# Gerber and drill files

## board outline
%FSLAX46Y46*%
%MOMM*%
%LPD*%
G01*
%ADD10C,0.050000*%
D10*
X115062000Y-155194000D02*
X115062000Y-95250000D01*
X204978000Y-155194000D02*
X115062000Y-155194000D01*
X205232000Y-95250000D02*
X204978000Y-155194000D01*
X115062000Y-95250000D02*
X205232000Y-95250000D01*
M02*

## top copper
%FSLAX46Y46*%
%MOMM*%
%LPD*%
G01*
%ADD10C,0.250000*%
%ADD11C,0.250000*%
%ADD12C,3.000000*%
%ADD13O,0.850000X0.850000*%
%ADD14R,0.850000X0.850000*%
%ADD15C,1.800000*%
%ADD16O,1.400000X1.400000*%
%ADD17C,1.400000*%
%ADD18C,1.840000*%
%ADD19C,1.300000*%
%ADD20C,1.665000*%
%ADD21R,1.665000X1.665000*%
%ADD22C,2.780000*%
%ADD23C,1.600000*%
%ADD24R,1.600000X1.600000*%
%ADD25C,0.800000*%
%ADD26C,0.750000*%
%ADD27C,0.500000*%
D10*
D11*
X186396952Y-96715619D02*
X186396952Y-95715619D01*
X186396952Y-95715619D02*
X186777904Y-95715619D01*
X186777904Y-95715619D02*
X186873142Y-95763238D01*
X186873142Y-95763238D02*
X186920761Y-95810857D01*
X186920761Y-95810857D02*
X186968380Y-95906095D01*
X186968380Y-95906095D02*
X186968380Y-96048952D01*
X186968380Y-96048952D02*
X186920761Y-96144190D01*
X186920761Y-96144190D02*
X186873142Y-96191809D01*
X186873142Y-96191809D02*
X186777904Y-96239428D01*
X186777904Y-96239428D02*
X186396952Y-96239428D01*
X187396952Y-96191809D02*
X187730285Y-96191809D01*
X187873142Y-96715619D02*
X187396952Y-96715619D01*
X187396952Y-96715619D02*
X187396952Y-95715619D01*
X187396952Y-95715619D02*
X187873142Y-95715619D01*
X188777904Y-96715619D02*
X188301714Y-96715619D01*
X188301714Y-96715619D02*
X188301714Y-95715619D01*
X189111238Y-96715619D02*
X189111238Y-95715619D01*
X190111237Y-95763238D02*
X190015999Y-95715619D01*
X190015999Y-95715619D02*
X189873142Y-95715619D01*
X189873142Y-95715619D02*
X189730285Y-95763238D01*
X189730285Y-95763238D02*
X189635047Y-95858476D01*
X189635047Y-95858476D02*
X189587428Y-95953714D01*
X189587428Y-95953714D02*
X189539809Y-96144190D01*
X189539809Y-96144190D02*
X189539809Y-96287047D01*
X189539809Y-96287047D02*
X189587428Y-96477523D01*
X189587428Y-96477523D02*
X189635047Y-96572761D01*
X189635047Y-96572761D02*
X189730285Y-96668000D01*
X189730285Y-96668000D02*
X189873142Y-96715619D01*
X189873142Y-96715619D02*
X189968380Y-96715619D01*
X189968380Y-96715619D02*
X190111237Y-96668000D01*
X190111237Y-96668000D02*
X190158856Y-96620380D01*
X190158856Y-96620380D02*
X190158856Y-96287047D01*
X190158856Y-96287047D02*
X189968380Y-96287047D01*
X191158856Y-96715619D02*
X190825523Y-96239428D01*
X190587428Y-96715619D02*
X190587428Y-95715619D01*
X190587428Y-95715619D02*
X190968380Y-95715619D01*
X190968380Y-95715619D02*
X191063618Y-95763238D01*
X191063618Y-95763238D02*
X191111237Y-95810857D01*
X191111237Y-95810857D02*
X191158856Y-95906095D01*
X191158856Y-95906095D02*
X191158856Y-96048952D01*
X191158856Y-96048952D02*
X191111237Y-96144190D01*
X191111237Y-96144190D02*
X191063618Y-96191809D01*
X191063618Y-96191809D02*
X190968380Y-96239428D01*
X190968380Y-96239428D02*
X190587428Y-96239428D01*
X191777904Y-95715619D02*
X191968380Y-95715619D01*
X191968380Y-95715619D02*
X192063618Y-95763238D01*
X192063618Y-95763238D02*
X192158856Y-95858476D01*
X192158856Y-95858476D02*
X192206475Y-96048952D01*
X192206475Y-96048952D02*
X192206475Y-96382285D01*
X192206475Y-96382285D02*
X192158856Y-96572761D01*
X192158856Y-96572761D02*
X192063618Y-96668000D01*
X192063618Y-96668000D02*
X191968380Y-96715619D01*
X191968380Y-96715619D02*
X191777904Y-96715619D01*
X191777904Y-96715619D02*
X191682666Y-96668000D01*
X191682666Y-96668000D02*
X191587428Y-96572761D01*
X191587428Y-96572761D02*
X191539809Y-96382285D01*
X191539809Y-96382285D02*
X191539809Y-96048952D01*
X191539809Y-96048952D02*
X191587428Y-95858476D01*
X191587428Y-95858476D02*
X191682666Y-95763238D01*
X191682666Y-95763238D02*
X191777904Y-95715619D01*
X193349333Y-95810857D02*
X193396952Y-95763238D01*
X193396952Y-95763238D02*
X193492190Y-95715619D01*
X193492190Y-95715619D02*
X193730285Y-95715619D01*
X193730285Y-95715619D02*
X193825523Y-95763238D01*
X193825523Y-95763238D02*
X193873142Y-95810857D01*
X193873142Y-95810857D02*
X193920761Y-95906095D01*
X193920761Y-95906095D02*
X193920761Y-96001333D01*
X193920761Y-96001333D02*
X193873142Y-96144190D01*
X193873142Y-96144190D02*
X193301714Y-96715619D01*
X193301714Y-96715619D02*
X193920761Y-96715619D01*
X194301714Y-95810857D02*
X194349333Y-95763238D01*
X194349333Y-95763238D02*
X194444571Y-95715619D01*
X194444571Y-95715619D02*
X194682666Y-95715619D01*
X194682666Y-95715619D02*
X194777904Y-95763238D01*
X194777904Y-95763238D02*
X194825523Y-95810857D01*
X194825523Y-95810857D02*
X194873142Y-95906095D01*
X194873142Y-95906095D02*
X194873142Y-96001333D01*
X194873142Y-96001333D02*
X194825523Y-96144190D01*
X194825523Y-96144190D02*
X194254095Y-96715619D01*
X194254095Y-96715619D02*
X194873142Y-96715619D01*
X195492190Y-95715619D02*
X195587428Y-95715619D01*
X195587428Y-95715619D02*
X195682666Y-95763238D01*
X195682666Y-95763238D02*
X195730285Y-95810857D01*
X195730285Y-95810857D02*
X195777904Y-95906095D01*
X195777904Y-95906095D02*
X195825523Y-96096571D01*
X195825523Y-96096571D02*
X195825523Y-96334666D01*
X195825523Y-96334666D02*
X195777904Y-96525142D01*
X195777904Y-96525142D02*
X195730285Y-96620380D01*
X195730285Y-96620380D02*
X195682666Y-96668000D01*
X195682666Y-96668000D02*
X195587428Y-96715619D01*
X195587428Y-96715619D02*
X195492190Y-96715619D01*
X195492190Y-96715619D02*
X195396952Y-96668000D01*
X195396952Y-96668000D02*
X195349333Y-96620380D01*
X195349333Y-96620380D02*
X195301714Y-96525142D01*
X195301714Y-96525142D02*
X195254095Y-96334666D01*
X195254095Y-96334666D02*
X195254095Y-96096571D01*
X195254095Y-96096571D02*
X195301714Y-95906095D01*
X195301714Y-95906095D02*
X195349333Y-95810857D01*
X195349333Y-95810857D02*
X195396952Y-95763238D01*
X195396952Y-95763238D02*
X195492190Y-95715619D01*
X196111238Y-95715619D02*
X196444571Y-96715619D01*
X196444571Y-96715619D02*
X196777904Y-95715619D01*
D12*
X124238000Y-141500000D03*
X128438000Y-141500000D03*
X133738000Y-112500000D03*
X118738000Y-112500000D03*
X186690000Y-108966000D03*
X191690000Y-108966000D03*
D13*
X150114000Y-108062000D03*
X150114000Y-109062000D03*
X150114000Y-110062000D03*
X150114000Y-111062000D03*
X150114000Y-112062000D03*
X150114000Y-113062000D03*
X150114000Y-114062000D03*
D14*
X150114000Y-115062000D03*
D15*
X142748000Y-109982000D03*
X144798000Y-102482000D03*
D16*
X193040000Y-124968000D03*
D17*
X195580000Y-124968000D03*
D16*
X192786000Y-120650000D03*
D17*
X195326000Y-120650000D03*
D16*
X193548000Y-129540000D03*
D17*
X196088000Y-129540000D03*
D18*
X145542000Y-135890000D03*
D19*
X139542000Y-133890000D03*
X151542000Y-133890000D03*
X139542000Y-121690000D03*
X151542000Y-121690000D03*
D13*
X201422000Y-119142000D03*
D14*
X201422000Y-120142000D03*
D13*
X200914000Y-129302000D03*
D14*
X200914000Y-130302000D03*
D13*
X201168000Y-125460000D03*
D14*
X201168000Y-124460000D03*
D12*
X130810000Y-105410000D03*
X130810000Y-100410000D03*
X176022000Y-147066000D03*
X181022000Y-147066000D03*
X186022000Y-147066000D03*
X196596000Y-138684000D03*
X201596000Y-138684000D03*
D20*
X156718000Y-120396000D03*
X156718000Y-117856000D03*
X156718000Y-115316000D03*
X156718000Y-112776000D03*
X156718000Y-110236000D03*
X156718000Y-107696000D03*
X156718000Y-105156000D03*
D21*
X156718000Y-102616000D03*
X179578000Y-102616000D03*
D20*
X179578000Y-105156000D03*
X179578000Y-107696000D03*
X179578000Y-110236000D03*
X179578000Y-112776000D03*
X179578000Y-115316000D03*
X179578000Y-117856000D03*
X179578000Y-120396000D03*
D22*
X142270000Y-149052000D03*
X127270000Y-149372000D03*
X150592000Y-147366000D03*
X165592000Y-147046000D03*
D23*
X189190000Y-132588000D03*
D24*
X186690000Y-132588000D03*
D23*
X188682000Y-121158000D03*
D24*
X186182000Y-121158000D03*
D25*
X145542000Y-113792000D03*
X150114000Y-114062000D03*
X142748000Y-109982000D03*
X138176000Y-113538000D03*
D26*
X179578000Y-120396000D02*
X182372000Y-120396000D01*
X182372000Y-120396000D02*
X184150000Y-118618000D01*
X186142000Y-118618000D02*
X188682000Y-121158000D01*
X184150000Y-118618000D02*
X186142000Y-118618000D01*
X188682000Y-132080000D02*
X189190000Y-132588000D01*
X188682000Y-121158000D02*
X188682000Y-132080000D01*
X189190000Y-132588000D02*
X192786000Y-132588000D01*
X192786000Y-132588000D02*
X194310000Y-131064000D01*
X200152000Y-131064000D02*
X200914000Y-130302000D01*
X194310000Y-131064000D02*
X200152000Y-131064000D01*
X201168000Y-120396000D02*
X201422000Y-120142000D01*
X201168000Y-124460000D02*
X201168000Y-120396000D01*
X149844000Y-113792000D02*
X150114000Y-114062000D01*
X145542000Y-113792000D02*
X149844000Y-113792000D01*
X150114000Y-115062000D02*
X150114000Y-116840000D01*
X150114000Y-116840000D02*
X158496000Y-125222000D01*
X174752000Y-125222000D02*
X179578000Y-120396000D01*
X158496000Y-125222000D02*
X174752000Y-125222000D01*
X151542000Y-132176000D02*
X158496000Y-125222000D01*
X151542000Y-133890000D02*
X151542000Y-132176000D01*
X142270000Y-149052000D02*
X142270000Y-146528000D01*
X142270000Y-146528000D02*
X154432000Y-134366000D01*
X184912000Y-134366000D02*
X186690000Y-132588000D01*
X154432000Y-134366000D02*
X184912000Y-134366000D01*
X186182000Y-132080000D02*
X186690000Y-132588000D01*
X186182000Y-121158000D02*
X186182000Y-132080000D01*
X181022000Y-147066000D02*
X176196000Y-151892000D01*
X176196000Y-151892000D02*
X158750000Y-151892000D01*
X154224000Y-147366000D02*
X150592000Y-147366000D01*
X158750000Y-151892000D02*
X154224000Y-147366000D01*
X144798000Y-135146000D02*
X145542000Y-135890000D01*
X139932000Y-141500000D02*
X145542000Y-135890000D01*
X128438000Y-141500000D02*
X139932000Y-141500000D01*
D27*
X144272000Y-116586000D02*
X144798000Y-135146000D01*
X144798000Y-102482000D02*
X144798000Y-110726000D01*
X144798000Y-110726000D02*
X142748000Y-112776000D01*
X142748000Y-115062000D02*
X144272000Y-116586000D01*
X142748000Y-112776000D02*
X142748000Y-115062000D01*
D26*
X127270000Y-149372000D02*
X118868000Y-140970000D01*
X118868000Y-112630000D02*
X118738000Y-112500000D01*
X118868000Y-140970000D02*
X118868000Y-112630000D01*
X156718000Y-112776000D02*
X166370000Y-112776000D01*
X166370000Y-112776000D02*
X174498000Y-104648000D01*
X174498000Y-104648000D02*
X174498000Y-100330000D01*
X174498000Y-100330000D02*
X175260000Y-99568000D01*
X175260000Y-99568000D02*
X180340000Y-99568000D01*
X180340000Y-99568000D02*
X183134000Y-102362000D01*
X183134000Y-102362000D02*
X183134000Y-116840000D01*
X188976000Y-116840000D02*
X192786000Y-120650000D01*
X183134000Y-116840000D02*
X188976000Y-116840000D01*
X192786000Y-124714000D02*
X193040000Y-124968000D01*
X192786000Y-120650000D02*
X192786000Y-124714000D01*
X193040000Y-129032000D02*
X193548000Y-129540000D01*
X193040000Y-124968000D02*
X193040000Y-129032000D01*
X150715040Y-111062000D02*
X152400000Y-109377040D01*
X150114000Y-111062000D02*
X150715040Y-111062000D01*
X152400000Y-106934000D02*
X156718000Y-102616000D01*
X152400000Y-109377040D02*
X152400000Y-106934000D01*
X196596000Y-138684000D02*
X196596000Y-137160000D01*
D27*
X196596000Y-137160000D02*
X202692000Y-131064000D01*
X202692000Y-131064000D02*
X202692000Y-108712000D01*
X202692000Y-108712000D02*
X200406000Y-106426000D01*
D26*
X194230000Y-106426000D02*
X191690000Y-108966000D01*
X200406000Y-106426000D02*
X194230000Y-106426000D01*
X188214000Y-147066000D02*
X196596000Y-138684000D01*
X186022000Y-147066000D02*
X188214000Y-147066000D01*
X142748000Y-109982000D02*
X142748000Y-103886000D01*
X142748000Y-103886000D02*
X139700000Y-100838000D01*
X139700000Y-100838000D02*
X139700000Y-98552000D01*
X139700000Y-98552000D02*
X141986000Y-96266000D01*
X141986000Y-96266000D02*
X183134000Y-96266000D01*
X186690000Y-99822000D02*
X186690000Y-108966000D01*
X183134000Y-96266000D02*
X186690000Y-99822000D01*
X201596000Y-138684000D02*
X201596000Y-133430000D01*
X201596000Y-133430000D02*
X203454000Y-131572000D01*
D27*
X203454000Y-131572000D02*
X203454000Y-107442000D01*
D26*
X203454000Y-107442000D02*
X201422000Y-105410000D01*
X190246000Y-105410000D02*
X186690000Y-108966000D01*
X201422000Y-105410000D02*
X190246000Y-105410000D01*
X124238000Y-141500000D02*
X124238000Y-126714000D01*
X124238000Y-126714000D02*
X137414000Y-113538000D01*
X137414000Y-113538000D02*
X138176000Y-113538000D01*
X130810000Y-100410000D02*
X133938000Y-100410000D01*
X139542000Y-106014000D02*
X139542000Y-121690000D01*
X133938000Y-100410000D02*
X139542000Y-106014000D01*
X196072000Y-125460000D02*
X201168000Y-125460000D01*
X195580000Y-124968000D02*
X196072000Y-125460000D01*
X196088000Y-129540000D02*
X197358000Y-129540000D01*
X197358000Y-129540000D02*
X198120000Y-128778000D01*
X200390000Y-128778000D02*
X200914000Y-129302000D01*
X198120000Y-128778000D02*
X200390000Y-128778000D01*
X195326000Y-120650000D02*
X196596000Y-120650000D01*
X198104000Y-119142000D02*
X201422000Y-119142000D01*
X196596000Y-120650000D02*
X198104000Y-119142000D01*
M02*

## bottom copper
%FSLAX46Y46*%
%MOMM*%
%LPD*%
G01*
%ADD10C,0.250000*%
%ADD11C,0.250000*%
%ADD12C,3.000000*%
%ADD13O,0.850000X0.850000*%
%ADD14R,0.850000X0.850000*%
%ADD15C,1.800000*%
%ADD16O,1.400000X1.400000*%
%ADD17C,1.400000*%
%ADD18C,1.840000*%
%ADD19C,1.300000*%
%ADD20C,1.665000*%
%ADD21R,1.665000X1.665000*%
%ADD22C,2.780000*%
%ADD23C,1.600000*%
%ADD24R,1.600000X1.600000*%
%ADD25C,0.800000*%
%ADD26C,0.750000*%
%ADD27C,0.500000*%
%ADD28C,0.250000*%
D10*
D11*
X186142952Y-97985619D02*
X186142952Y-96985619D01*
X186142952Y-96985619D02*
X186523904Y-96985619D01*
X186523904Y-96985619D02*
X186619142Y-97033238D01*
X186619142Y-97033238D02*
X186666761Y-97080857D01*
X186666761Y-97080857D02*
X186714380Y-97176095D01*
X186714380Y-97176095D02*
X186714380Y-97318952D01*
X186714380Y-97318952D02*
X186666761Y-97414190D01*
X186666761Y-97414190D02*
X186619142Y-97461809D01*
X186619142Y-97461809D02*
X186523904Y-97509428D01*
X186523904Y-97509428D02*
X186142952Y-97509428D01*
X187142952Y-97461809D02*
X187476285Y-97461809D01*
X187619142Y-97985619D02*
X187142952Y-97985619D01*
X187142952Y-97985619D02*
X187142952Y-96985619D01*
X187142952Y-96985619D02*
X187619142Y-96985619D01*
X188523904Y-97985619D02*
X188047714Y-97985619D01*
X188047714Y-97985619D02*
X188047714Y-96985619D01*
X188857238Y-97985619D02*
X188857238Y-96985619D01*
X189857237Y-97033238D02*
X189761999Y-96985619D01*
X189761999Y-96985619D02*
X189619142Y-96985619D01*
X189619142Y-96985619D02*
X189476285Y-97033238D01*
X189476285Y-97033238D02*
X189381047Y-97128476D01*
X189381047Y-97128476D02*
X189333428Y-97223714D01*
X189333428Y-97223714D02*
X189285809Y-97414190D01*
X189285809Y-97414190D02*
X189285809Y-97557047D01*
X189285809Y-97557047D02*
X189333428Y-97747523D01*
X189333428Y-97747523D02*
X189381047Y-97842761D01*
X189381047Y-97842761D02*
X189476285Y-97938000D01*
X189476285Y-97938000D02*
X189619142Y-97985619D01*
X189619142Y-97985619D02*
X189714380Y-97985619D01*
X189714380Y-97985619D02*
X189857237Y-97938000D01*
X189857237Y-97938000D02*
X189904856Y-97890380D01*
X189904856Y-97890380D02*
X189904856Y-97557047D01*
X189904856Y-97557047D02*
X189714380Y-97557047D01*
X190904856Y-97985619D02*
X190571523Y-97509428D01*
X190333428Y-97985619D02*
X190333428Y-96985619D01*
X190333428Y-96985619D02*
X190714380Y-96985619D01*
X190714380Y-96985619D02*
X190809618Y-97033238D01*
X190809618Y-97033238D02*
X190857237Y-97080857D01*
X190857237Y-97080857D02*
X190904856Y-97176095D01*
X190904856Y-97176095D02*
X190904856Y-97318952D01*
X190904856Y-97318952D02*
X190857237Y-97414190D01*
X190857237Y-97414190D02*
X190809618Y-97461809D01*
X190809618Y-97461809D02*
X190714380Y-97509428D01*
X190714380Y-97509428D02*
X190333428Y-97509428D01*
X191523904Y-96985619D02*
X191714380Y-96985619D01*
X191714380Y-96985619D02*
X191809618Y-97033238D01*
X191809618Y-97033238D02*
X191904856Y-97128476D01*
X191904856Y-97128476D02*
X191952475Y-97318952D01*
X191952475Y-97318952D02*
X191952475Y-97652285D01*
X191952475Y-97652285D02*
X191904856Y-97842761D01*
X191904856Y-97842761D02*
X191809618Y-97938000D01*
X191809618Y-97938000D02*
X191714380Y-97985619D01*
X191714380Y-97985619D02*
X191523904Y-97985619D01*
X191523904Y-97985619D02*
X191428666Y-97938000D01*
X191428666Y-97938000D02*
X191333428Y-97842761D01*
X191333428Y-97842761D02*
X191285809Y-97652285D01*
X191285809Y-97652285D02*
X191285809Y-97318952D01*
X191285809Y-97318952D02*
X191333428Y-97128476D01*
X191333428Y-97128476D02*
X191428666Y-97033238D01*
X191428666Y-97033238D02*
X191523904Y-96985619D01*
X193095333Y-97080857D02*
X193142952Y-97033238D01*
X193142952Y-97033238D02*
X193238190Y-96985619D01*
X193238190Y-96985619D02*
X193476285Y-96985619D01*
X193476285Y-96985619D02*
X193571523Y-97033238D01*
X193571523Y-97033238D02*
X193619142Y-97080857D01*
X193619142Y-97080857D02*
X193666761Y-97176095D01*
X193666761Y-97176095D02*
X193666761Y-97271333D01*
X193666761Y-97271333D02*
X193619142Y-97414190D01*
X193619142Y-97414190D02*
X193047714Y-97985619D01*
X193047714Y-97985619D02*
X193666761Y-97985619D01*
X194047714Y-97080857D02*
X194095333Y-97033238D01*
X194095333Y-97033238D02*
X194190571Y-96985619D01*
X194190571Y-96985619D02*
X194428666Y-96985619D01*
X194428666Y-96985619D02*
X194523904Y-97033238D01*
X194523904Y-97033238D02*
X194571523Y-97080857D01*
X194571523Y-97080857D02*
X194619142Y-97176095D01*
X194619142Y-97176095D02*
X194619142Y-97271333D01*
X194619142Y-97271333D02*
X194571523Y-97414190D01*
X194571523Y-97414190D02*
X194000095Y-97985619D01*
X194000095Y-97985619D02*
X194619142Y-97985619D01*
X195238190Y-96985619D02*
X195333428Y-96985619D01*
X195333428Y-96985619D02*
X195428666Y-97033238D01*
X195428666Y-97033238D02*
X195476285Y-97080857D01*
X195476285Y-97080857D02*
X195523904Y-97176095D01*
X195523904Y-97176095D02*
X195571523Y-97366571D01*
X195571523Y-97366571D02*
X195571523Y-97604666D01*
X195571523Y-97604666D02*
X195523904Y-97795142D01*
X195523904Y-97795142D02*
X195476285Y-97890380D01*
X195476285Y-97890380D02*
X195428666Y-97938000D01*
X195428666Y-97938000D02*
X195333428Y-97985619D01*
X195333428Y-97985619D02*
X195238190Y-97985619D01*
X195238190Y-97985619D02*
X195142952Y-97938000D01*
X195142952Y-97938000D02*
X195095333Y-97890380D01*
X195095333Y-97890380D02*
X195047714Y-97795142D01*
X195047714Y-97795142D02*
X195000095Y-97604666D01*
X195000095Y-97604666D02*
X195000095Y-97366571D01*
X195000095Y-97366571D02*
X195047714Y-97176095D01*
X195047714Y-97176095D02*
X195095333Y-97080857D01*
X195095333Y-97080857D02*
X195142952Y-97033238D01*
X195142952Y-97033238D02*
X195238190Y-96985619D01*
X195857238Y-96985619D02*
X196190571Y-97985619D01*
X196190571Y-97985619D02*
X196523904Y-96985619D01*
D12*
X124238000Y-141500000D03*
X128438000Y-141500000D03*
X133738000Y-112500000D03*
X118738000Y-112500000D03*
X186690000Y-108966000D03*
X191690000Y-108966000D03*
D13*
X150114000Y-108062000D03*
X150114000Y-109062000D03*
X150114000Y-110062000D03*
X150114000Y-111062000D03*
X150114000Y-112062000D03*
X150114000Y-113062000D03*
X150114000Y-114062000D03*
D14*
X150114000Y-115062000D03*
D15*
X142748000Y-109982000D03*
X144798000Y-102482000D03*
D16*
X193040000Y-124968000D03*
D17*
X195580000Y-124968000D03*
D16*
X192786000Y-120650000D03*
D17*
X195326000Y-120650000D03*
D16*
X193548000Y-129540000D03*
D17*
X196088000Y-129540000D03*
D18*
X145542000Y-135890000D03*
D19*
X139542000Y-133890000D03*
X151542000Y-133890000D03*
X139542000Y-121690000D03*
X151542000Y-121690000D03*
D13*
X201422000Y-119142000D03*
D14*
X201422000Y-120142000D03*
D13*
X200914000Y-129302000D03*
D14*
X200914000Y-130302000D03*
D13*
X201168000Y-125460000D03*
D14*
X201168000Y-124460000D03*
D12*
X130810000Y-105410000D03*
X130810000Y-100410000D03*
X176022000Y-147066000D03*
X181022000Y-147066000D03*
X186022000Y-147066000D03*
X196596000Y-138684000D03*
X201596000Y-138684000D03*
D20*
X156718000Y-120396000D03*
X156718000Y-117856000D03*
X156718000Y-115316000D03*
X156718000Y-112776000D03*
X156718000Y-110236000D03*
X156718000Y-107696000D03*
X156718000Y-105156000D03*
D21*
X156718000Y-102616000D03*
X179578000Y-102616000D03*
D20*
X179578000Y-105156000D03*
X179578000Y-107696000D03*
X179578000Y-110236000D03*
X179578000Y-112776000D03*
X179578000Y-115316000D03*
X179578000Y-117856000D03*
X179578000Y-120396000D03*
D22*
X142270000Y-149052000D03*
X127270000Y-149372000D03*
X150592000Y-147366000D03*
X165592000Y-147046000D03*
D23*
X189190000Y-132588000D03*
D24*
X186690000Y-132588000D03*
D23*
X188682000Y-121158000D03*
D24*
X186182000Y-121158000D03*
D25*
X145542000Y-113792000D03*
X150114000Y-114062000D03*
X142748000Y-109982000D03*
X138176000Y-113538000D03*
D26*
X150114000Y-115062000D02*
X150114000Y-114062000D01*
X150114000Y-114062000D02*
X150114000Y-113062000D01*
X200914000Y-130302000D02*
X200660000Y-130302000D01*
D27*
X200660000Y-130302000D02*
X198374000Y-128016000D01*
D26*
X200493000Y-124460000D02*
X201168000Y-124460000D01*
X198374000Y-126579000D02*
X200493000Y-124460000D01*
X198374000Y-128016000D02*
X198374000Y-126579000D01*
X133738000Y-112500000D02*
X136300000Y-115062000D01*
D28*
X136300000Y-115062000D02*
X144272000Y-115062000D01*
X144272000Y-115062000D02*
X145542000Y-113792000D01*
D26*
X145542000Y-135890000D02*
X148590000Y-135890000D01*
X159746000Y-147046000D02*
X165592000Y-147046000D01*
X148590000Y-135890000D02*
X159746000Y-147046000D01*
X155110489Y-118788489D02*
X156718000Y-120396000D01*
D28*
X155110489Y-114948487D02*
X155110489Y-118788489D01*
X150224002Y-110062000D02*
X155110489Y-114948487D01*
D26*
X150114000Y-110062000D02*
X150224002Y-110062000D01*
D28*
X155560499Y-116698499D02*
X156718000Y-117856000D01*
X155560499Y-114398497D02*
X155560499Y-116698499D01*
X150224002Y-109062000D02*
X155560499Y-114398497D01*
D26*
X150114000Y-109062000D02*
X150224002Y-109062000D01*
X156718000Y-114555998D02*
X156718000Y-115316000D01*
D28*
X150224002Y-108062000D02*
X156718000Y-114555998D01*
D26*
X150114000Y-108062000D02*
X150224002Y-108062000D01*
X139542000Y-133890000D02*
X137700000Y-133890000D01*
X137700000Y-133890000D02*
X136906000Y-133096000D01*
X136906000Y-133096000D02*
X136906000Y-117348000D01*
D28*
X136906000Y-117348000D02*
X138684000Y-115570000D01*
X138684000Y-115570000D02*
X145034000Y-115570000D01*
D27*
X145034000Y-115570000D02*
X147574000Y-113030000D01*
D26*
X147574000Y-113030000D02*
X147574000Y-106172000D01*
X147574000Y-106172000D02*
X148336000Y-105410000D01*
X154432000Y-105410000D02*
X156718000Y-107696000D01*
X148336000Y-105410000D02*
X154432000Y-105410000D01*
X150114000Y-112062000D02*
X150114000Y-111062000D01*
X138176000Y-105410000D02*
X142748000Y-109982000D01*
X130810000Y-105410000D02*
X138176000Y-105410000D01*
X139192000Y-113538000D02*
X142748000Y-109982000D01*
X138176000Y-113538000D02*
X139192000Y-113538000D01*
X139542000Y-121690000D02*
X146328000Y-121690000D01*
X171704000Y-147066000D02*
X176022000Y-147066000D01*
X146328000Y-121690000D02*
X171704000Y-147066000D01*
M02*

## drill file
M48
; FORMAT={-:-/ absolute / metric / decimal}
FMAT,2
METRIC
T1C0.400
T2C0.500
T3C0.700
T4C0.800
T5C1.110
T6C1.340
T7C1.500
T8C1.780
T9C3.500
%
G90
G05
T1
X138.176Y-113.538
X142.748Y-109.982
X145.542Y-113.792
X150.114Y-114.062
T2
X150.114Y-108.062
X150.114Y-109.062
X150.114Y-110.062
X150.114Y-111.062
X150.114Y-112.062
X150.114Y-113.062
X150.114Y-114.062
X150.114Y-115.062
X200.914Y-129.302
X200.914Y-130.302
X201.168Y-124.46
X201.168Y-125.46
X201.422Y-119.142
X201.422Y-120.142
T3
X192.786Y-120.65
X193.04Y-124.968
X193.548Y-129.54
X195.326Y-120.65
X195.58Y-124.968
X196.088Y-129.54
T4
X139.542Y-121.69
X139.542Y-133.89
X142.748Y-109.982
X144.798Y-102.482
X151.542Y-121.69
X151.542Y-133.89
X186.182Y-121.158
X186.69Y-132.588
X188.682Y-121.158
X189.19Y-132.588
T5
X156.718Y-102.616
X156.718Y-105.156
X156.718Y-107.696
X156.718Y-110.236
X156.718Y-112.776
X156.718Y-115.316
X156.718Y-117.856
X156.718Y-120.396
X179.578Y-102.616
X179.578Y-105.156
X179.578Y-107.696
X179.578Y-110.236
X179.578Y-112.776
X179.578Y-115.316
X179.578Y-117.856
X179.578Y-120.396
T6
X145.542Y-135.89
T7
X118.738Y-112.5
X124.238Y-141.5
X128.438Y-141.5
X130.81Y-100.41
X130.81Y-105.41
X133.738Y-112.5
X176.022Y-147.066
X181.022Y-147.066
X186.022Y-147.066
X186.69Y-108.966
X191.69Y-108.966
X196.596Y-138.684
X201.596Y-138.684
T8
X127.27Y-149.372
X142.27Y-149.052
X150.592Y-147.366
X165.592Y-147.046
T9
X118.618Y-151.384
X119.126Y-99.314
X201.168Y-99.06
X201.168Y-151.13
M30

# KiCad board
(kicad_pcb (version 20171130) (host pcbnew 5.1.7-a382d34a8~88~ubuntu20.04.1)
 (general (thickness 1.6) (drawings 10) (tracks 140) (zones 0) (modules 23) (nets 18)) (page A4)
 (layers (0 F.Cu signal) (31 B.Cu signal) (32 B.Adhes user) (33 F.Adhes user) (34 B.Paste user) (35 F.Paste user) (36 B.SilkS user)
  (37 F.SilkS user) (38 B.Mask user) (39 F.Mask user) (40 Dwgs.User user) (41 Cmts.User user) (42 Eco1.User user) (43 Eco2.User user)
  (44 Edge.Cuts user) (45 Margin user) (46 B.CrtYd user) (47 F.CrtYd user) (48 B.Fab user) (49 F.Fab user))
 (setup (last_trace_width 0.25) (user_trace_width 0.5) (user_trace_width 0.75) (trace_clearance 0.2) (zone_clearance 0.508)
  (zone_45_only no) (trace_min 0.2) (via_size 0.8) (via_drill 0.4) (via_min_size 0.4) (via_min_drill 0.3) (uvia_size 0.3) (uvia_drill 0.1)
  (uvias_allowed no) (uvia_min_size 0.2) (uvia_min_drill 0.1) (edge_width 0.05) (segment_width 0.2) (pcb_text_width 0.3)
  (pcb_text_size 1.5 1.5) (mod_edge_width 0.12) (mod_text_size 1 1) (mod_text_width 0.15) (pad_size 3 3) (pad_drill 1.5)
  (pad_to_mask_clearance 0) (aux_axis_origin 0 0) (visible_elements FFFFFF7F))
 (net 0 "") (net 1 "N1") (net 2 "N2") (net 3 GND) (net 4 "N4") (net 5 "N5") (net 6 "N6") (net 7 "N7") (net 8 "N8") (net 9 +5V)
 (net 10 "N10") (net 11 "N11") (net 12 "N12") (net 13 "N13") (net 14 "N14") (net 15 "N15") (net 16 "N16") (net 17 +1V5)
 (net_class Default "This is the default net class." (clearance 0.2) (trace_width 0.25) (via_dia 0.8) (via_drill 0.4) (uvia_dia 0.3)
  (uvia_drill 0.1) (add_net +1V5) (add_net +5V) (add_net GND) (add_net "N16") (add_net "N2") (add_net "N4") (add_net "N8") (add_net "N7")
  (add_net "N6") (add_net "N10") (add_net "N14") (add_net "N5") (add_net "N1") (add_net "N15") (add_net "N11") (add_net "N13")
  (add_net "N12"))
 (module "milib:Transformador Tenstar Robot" (layer F.Cu) (at 126.238 127 90)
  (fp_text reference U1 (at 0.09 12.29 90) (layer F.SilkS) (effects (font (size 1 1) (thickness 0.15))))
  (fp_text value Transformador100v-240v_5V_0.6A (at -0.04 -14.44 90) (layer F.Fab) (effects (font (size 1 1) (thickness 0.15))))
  (pad 1 thru_hole circle (at -14.5 -2 90) (size 3 3) (drill oval 1.5) (layers *.Cu *.Mask) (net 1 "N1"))
  (pad 0 thru_hole circle (at -14.5 2.2 90) (size 3 3) (drill oval 1.5) (layers *.Cu *.Mask) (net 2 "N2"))
  (pad 3 thru_hole circle (at 14.5 7.5 90) (size 3 3) (drill oval 1.5) (layers *.Cu *.Mask) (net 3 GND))
  (pad 2 thru_hole circle (at 14.5 -7.5 90) (size 3 3) (drill oval 1.5) (layers *.Cu *.Mask) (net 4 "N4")))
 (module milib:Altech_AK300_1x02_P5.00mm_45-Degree (layer F.Cu) (at 186.69 108.966)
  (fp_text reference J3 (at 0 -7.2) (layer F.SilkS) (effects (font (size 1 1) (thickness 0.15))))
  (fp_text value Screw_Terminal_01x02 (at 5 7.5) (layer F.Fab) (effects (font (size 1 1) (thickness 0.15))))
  (pad 1 thru_hole circle (at 0 0) (size 3 3) (drill 1.5) (layers *.Cu *.Mask) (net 1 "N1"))
  (pad 2 thru_hole circle (at 5 0) (size 3 3) (drill 1.5) (layers *.Cu *.Mask) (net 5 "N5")))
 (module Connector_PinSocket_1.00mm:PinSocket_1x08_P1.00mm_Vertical (layer F.Cu) (at 150.114 115.062 180)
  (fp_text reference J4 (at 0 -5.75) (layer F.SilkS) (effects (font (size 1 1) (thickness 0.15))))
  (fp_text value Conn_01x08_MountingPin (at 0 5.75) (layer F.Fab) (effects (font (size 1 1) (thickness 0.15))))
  (pad 8 thru_hole oval (at 0 7 180) (size 0.85 0.85) (drill 0.5) (layers *.Cu *.Mask) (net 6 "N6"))
  (pad 7 thru_hole oval (at 0 6 180) (size 0.85 0.85) (drill 0.5) (layers *.Cu *.Mask) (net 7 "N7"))
  (pad 6 thru_hole oval (at 0 5 180) (size 0.85 0.85) (drill 0.5) (layers *.Cu *.Mask) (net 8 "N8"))
  (pad 5 thru_hole oval (at 0 4 180) (size 0.85 0.85) (drill 0.5) (layers *.Cu *.Mask) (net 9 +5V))
  (pad 4 thru_hole oval (at 0 3 180) (size 0.85 0.85) (drill 0.5) (layers *.Cu *.Mask) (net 9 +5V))
  (pad 3 thru_hole oval (at 0 2 180) (size 0.85 0.85) (drill 0.5) (layers *.Cu *.Mask) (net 3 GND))
  (pad 2 thru_hole oval (at 0 1 180) (size 0.85 0.85) (drill 0.5) (layers *.Cu *.Mask) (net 3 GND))
  (pad 1 thru_hole rect (at 0 0 180) (size 0.85 0.85) (drill 0.5) (layers *.Cu *.Mask) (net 3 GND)))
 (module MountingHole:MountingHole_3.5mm (layer F.Cu) (at 201.168 151.13)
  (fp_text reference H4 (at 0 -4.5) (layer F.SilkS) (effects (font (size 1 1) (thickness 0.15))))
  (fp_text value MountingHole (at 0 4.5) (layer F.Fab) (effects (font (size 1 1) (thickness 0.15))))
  (pad 1 np_thru_hole circle (at 0 0) (size 3.5 3.5) (drill 3.5) (layers *.Cu *.Mask)))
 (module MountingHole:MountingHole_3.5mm (layer F.Cu) (at 201.168 99.06)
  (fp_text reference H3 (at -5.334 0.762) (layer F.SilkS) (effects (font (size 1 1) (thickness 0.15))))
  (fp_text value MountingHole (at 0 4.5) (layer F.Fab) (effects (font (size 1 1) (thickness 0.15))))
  (pad 1 np_thru_hole circle (at 0 0) (size 3.5 3.5) (drill 3.5) (layers *.Cu *.Mask)))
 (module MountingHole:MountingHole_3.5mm (layer F.Cu) (at 118.618 151.384)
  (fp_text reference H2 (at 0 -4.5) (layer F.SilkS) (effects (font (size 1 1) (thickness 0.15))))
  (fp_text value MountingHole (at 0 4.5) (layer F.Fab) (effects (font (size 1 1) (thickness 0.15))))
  (pad 1 np_thru_hole circle (at 0 0) (size 3.5 3.5) (drill 3.5) (layers *.Cu *.Mask)))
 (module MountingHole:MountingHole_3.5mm (layer F.Cu) (at 119.126 99.314)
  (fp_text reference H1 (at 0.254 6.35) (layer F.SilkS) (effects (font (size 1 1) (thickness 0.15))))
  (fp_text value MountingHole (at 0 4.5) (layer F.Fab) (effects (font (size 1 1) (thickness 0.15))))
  (pad 1 np_thru_hole circle (at 0 0) (size 3.5 3.5) (drill 3.5) (layers *.Cu *.Mask)))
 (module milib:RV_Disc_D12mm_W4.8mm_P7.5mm (layer F.Cu) (at 142.748 109.982 90)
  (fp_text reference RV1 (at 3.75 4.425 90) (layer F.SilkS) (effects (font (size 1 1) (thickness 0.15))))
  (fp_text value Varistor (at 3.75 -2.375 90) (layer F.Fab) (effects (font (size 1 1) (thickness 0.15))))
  (pad 1 thru_hole circle (at 0 0 90) (size 1.8 1.8) (drill 0.8) (layers *.Cu *.Mask) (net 1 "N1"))
  (pad 2 thru_hole circle (at 7.5 2.05 90) (size 1.8 1.8) (drill 0.8) (layers *.Cu *.Mask) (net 2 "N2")))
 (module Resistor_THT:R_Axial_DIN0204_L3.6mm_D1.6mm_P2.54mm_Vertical (layer F.Cu) (at 195.58 124.968 180)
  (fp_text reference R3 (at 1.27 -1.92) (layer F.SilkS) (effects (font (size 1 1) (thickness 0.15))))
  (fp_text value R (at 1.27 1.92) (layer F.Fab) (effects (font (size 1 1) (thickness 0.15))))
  (pad 2 thru_hole oval (at 2.54 0 180) (size 1.4 1.4) (drill 0.7) (layers *.Cu *.Mask) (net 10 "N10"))
  (pad 1 thru_hole circle (at 0 0 180) (size 1.4 1.4) (drill 0.7) (layers *.Cu *.Mask) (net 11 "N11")))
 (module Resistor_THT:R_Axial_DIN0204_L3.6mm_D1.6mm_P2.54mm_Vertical (layer F.Cu) (at 195.326 120.65 180)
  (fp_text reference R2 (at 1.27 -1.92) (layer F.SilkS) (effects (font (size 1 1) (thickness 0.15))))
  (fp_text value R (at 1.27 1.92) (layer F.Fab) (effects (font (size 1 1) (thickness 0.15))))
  (pad 2 thru_hole oval (at 2.54 0 180) (size 1.4 1.4) (drill 0.7) (layers *.Cu *.Mask) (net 10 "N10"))
  (pad 1 thru_hole circle (at 0 0 180) (size 1.4 1.4) (drill 0.7) (layers *.Cu *.Mask) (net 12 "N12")))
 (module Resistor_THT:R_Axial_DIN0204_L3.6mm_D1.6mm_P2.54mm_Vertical (layer F.Cu) (at 196.088 129.54 180)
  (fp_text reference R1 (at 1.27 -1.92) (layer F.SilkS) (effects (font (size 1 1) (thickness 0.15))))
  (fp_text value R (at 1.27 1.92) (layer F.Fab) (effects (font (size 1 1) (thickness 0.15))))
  (pad 2 thru_hole oval (at 2.54 0 180) (size 1.4 1.4) (drill 0.7) (layers *.Cu *.Mask) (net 10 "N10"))
  (pad 1 thru_hole circle (at 0 0 180) (size 1.4 1.4) (drill 0.7) (layers *.Cu *.Mask) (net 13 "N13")))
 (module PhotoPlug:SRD (layer F.Cu) (at 145.542 135.89 90)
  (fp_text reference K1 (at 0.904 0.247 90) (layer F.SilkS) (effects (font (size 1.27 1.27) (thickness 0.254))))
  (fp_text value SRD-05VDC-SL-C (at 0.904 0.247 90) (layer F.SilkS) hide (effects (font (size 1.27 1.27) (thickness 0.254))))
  (pad 1 thru_hole circle (at 0 0 90) (size 1.84 1.84) (drill 1.34) (layers *.Cu *.Mask) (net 2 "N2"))
  (pad 2 thru_hole circle (at 2 -6 90) (size 1.3 1.3) (drill 0.8) (layers *.Cu *.Mask) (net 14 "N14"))
  (pad 3 thru_hole circle (at 2 6 90) (size 1.3 1.3) (drill 0.8) (layers *.Cu *.Mask) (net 3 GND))
  (pad 4 thru_hole circle (at 14.2 -6 90) (size 1.3 1.3) (drill 0.8) (layers *.Cu *.Mask) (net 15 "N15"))
  (pad 5 thru_hole circle (at 14.2 6 90) (size 1.3 1.3) (drill 0.8) (layers *.Cu *.Mask)))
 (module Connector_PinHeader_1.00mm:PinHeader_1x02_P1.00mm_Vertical (layer F.Cu) (at 201.422 120.142 180)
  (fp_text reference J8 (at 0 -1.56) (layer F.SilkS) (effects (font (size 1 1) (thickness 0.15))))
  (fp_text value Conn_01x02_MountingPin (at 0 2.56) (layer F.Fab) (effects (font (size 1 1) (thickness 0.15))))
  (pad 2 thru_hole oval (at 0 1 180) (size 0.85 0.85) (drill 0.5) (layers *.Cu *.Mask) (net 12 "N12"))
  (pad 1 thru_hole rect (at 0 0 180) (size 0.85 0.85) (drill 0.5) (layers *.Cu *.Mask) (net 3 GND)))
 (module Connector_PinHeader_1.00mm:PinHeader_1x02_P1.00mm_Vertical (layer F.Cu) (at 200.914 130.302 180)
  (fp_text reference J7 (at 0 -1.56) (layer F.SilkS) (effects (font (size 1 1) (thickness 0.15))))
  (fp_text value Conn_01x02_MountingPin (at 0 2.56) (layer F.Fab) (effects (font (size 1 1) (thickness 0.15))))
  (pad 2 thru_hole oval (at 0 1 180) (size 0.85 0.85) (drill 0.5) (layers *.Cu *.Mask) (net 13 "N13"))
  (pad 1 thru_hole rect (at 0 0 180) (size 0.85 0.85) (drill 0.5) (layers *.Cu *.Mask) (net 3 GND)))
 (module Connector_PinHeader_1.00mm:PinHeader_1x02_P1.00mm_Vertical (layer F.Cu) (at 201.168 124.46)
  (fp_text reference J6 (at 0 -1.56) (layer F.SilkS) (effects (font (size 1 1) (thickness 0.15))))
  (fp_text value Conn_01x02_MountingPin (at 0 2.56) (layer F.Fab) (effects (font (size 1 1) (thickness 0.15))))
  (pad 2 thru_hole oval (at 0 1) (size 0.85 0.85) (drill 0.5) (layers *.Cu *.Mask) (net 11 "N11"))
  (pad 1 thru_hole rect (at 0 0) (size 0.85 0.85) (drill 0.5) (layers *.Cu *.Mask) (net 3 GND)))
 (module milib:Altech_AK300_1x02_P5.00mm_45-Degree (layer F.Cu) (at 130.81 105.41 90)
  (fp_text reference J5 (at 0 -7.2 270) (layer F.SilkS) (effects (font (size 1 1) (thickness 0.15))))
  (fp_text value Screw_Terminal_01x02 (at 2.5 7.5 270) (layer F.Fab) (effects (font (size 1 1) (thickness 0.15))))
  (pad 1 thru_hole circle (at 0 0 90) (size 3 3) (drill 1.5) (layers *.Cu *.Mask) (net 1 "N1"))
  (pad 2 thru_hole circle (at 5 0 90) (size 3 3) (drill 1.5) (layers *.Cu *.Mask) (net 15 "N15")))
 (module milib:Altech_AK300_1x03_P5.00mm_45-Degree (layer F.Cu) (at 176.022 147.066)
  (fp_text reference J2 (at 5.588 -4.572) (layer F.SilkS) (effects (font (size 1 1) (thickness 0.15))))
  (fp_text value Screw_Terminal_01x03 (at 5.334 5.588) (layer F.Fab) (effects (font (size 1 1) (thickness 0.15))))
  (pad 1 thru_hole circle (at 0 0) (size 3 3) (drill oval 1.5) (layers *.Cu *.Mask) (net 15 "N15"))
  (pad 2 thru_hole circle (at 5 0) (size 3 3) (drill 1.5) (layers *.Cu *.Mask) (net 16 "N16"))
  (pad 3 thru_hole circle (at 10 0) (size 3 3) (drill oval 1.5) (layers *.Cu *.Mask) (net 5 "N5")))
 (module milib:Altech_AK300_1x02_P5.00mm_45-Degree (layer F.Cu) (at 196.596 138.684)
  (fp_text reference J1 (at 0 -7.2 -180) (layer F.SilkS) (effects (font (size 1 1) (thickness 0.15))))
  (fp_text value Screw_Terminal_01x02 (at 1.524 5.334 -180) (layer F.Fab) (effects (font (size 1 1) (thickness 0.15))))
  (pad 1 thru_hole circle (at 0 0) (size 3 3) (drill 1.5) (layers *.Cu *.Mask) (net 5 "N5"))
  (pad 2 thru_hole circle (at 5 0) (size 3 3) (drill 1.5) (layers *.Cu *.Mask) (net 1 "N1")))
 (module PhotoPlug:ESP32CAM (layer F.Cu) (at 156.718 120.396)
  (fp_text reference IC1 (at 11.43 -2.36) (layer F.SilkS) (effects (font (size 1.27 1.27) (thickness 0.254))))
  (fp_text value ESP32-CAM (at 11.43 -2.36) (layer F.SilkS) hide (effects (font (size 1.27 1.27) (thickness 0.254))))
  (pad 1 thru_hole circle (at 0 0) (size 1.665 1.665) (drill 1.11) (layers *.Cu *.Mask) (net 8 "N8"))
  (pad 2 thru_hole circle (at 0 -2.54) (size 1.665 1.665) (drill 1.11) (layers *.Cu *.Mask) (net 7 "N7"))
  (pad 3 thru_hole circle (at 0 -5.08) (size 1.665 1.665) (drill 1.11) (layers *.Cu *.Mask) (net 6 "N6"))
  (pad 4 thru_hole circle (at 0 -7.62) (size 1.665 1.665) (drill 1.11) (layers *.Cu *.Mask) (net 10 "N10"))
  (pad 5 thru_hole circle (at 0 -10.16) (size 1.665 1.665) (drill 1.11) (layers *.Cu *.Mask))
  (pad 6 thru_hole circle (at 0 -12.7) (size 1.665 1.665) (drill 1.11) (layers *.Cu *.Mask) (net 14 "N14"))
  (pad 7 thru_hole circle (at 0 -15.24) (size 1.665 1.665) (drill 1.11) (layers *.Cu *.Mask))
  (pad 8 thru_hole rect (at 0 -17.78) (size 1.665 1.665) (drill 1.11) (layers *.Cu *.Mask) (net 9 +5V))
  (pad 9 thru_hole rect (at 22.86 -17.78) (size 1.665 1.665) (drill 1.11) (layers *.Cu *.Mask))
  (pad 10 thru_hole circle (at 22.86 -15.24) (size 1.665 1.665) (drill 1.11) (layers *.Cu *.Mask))
  (pad 11 thru_hole circle (at 22.86 -12.7) (size 1.665 1.665) (drill 1.11) (layers *.Cu *.Mask))
  (pad 12 thru_hole circle (at 22.86 -10.16) (size 1.665 1.665) (drill 1.11) (layers *.Cu *.Mask))
  (pad 13 thru_hole circle (at 22.86 -7.62) (size 1.665 1.665) (drill 1.11) (layers *.Cu *.Mask))
  (pad 14 thru_hole circle (at 22.86 -5.08) (size 1.665 1.665) (drill 1.11) (layers *.Cu *.Mask))
  (pad 15 thru_hole circle (at 22.86 -2.54) (size 1.665 1.665) (drill 1.11) (layers *.Cu *.Mask))
  (pad 16 thru_hole circle (at 22.86 0) (size 1.665 1.665) (drill 1.11) (layers *.Cu *.Mask) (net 3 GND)))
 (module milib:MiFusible (layer F.Cu) (at 134.62 149.352 180)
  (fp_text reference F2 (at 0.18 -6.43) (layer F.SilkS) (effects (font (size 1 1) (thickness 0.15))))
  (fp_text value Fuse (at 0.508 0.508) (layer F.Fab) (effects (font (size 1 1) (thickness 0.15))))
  (pad 1 thru_hole circle (at -7.65 0.3 180) (size 2.78 2.78) (drill 1.78) (layers *.Cu *.Mask) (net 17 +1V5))
  (pad 2 thru_hole circle (at 7.35 -0.02 180) (size 2.78 2.78) (drill 1.78) (layers *.Cu *.Mask) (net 4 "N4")))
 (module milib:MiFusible (layer F.Cu) (at 158.242 147.066)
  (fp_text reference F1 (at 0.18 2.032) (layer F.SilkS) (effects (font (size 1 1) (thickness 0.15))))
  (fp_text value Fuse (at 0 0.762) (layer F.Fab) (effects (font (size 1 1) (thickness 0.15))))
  (pad 1 thru_hole circle (at -7.65 0.3) (size 2.78 2.78) (drill 1.78) (layers *.Cu *.Mask) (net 16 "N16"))
  (pad 2 thru_hole circle (at 7.35 -0.02) (size 2.78 2.78) (drill 1.78) (layers *.Cu *.Mask) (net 2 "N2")))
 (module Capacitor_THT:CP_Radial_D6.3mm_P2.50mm (layer F.Cu) (at 186.69 132.588)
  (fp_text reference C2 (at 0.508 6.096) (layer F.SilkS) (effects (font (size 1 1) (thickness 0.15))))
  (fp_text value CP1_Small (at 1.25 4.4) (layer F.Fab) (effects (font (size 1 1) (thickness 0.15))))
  (pad 2 thru_hole circle (at 2.5 0) (size 1.6 1.6) (drill 0.8) (layers *.Cu *.Mask) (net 3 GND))
  (pad 1 thru_hole rect (at 0 0) (size 1.6 1.6) (drill 0.8) (layers *.Cu *.Mask) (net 17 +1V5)))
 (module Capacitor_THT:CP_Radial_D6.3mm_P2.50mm (layer F.Cu) (at 186.182 121.158)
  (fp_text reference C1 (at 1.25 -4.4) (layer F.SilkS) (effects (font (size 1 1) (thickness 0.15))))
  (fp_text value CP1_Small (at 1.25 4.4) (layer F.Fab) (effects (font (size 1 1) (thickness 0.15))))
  (pad 2 thru_hole circle (at 2.5 0) (size 1.6 1.6) (drill 0.8) (layers *.Cu *.Mask) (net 3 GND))
  (pad 1 thru_hole rect (at 0 0) (size 1.6 1.6) (drill 0.8) (layers *.Cu *.Mask) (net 17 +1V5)))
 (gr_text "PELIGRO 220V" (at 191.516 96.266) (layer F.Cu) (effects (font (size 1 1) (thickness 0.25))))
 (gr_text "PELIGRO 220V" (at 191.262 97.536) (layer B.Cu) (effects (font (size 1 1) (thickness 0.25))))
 (gr_line (start 115.062 155.194) (end 115.062 95.25) (layer Edge.Cuts) (width 0.05))
 (gr_line (start 204.978 155.194) (end 115.062 155.194) (layer Edge.Cuts) (width 0.05))
 (gr_line (start 205.232 95.25) (end 204.978 155.194) (layer Edge.Cuts) (width 0.05))
 (gr_line (start 115.062 95.25) (end 205.232 95.25) (layer Edge.Cuts) (width 0.05))
 (segment (start 150.114 115.062) (end 150.114 114.062) (width 0.75) (layer B.Cu) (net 3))
 (segment (start 150.114 114.062) (end 150.114 113.062) (width 0.75) (layer B.Cu) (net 3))
 (segment (start 179.578 120.396) (end 182.372 120.396) (width 0.75) (layer F.Cu) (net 3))
 (segment (start 182.372 120.396) (end 184.15 118.618) (width 0.75) (layer F.Cu) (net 3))
 (segment (start 186.142 118.618) (end 188.682 121.158) (width 0.75) (layer F.Cu) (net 3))
 (segment (start 184.15 118.618) (end 186.142 118.618) (width 0.75) (layer F.Cu) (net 3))
 (segment (start 188.682 132.08) (end 189.19 132.588) (width 0.75) (layer F.Cu) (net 3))
 (segment (start 188.682 121.158) (end 188.682 132.08) (width 0.75) (layer F.Cu) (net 3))
 (segment (start 189.19 132.588) (end 192.786 132.588) (width 0.75) (layer F.Cu) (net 3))
 (segment (start 192.786 132.588) (end 194.31 131.064) (width 0.75) (layer F.Cu) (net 3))
 (segment (start 200.152 131.064) (end 200.914 130.302) (width 0.75) (layer F.Cu) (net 3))
 (segment (start 194.31 131.064) (end 200.152 131.064) (width 0.75) (layer F.Cu) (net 3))
 (segment (start 200.914 130.302) (end 200.66 130.302) (width 0.75) (layer B.Cu) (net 3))
 (segment (start 200.66 130.302) (end 198.374 128.016) (width 0.5) (layer B.Cu) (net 3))
 (segment (start 200.493 124.46) (end 201.168 124.46) (width 0.75) (layer B.Cu) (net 3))
 (segment (start 198.374 126.579) (end 200.493 124.46) (width 0.75) (layer B.Cu) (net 3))
 (segment (start 198.374 128.016) (end 198.374 126.579) (width 0.75) (layer B.Cu) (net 3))
 (segment (start 201.168 120.396) (end 201.422 120.142) (width 0.75) (layer F.Cu) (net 3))
 (segment (start 201.168 124.46) (end 201.168 120.396) (width 0.75) (layer F.Cu) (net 3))
 (segment (start 133.738 112.5) (end 136.3 115.062) (width 0.75) (layer B.Cu) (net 3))
 (segment (start 136.3 115.062) (end 144.272 115.062) (width 0.25) (layer B.Cu) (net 3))
 (via (at 145.542 113.792) (size 0.8) (drill 0.4) (layers F.Cu B.Cu) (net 3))
 (segment (start 144.272 115.062) (end 145.542 113.792) (width 0.25) (layer B.Cu) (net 3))
 (via (at 150.114 114.062) (size 0.8) (drill 0.4) (layers F.Cu B.Cu) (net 3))
 (segment (start 149.844 113.792) (end 150.114 114.062) (width 0.75) (layer F.Cu) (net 3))
 (segment (start 145.542 113.792) (end 149.844 113.792) (width 0.75) (layer F.Cu) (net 3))
 (segment (start 150.114 115.062) (end 150.114 116.84) (width 0.75) (layer F.Cu) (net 3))
 (segment (start 150.114 116.84) (end 158.496 125.222) (width 0.75) (layer F.Cu) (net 3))
 (segment (start 174.752 125.222) (end 179.578 120.396) (width 0.75) (layer F.Cu) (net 3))
 (segment (start 158.496 125.222) (end 174.752 125.222) (width 0.75) (layer F.Cu) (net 3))
 (segment (start 151.542 132.176) (end 158.496 125.222) (width 0.75) (layer F.Cu) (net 3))
 (segment (start 151.542 133.89) (end 151.542 132.176) (width 0.75) (layer F.Cu) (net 3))
 (segment (start 142.27 149.052) (end 142.27 146.528) (width 0.75) (layer F.Cu) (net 17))
 (segment (start 142.27 146.528) (end 154.432 134.366) (width 0.75) (layer F.Cu) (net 17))
 (segment (start 184.912 134.366) (end 186.69 132.588) (width 0.75) (layer F.Cu) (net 17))
 (segment (start 154.432 134.366) (end 184.912 134.366) (width 0.75) (layer F.Cu) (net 17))
 (segment (start 186.182 132.08) (end 186.69 132.588) (width 0.75) (layer F.Cu) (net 17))
 (segment (start 186.182 121.158) (end 186.182 132.08) (width 0.75) (layer F.Cu) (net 17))
 (segment (start 181.022 147.066) (end 176.196 151.892) (width 0.75) (layer F.Cu) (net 16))
 (segment (start 176.196 151.892) (end 158.75 151.892) (width 0.75) (layer F.Cu) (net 16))
 (segment (start 154.224 147.366) (end 150.592 147.366) (width 0.75) (layer F.Cu) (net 16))
 (segment (start 158.75 151.892) (end 154.224 147.366) (width 0.75) (layer F.Cu) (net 16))
 (segment (start 145.542 135.89) (end 148.59 135.89) (width 0.75) (layer B.Cu) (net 2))
 (segment (start 159.746 147.046) (end 165.592 147.046) (width 0.75) (layer B.Cu) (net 2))
 (segment (start 148.59 135.89) (end 159.746 147.046) (width 0.75) (layer B.Cu) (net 2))
 (segment (start 144.798 135.146) (end 145.542 135.89) (width 0.75) (layer F.Cu) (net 2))
 (segment (start 139.932 141.5) (end 145.542 135.89) (width 0.75) (layer F.Cu) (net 2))
 (segment (start 128.438 141.5) (end 139.932 141.5) (width 0.75) (layer F.Cu) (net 2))
 (segment (start 144.272 116.586) (end 144.798 135.146) (width 0.5) (layer F.Cu) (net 2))
 (segment (start 144.798 102.482) (end 144.798 110.726) (width 0.5) (layer F.Cu) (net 2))
 (segment (start 144.798 110.726) (end 142.748 112.776) (width 0.5) (layer F.Cu) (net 2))
 (segment (start 142.748 115.062) (end 144.272 116.586) (width 0.5) (layer F.Cu) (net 2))
 (segment (start 142.748 112.776) (end 142.748 115.062) (width 0.5) (layer F.Cu) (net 2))
 (segment (start 127.27 149.372) (end 118.868 140.97) (width 0.75) (layer F.Cu) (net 4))
 (segment (start 118.868 112.63) (end 118.738 112.5) (width 0.75) (layer F.Cu) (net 4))
 (segment (start 118.868 140.97) (end 118.868 112.63) (width 0.75) (layer F.Cu) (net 4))
 (segment (start 155.110489 118.788489) (end 156.718 120.396) (width 0.75) (layer B.Cu) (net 8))
 (segment (start 155.110489 114.948487) (end 155.110489 118.788489) (width 0.25) (layer B.Cu) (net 8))
 (segment (start 150.224002 110.062) (end 155.110489 114.948487) (width 0.25) (layer B.Cu) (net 8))
 (segment (start 150.114 110.062) (end 150.224002 110.062) (width 0.75) (layer B.Cu) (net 8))
 (segment (start 155.560499 116.698499) (end 156.718 117.856) (width 0.25) (layer B.Cu) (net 7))
 (segment (start 155.560499 114.398497) (end 155.560499 116.698499) (width 0.25) (layer B.Cu) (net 7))
 (segment (start 150.224002 109.062) (end 155.560499 114.398497) (width 0.25) (layer B.Cu) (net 7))
 (segment (start 150.114 109.062) (end 150.224002 109.062) (width 0.75) (layer B.Cu) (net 7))
 (segment (start 156.718 114.555998) (end 156.718 115.316) (width 0.75) (layer B.Cu) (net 6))
 (segment (start 150.224002 108.062) (end 156.718 114.555998) (width 0.25) (layer B.Cu) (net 6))
 (segment (start 150.114 108.062) (end 150.224002 108.062) (width 0.75) (layer B.Cu) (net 6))
 (segment (start 156.718 112.776) (end 166.37 112.776) (width 0.75) (layer F.Cu) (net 10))
 (segment (start 166.37 112.776) (end 174.498 104.648) (width 0.75) (layer F.Cu) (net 10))
 (segment (start 174.498 104.648) (end 174.498 100.33) (width 0.75) (layer F.Cu) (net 10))
 (segment (start 174.498 100.33) (end 175.26 99.568) (width 0.75) (layer F.Cu) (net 10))
 (segment (start 175.26 99.568) (end 180.34 99.568) (width 0.75) (layer F.Cu) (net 10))
 (segment (start 180.34 99.568) (end 183.134 102.362) (width 0.75) (layer F.Cu) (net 10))
 (segment (start 183.134 102.362) (end 183.134 116.84) (width 0.75) (layer F.Cu) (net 10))
 (segment (start 188.976 116.84) (end 192.786 120.65) (width 0.75) (layer F.Cu) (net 10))
 (segment (start 183.134 116.84) (end 188.976 116.84) (width 0.75) (layer F.Cu) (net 10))
 (segment (start 192.786 124.714) (end 193.04 124.968) (width 0.75) (layer F.Cu) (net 10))
 (segment (start 192.786 120.65) (end 192.786 124.714) (width 0.75) (layer F.Cu) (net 10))
 (segment (start 193.04 129.032) (end 193.548 129.54) (width 0.75) (layer F.Cu) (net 10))
 (segment (start 193.04 124.968) (end 193.04 129.032) (width 0.75) (layer F.Cu) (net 10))
 (segment (start 139.542 133.89) (end 137.7 133.89) (width 0.75) (layer B.Cu) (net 14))
 (segment (start 137.7 133.89) (end 136.906 133.096) (width 0.75) (layer B.Cu) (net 14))
 (segment (start 136.906 133.096) (end 136.906 117.348) (width 0.75) (layer B.Cu) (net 14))
 (segment (start 136.906 117.348) (end 138.684 115.57) (width 0.25) (layer B.Cu) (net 14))
 (segment (start 138.684 115.57) (end 145.034 115.57) (width 0.25) (layer B.Cu) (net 14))
 (segment (start 145.034 115.57) (end 147.574 113.03) (width 0.5) (layer B.Cu) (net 14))
 (segment (start 147.574 113.03) (end 147.574 106.172) (width 0.75) (layer B.Cu) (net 14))
 (segment (start 147.574 106.172) (end 148.336 105.41) (width 0.75) (layer B.Cu) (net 14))
 (segment (start 154.432 105.41) (end 156.718 107.696) (width 0.75) (layer B.Cu) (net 14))
 (segment (start 148.336 105.41) (end 154.432 105.41) (width 0.75) (layer B.Cu) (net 14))
 (segment (start 150.71504 111.062) (end 152.4 109.37704) (width 0.75) (layer F.Cu) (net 9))
 (segment (start 150.114 111.062) (end 150.71504 111.062) (width 0.75) (layer F.Cu) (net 9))
 (segment (start 152.4 106.934) (end 156.718 102.616) (width 0.75) (layer F.Cu) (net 9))
 (segment (start 152.4 109.37704) (end 152.4 106.934) (width 0.75) (layer F.Cu) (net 9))
 (segment (start 150.114 112.062) (end 150.114 111.062) (width 0.75) (layer B.Cu) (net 9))
 (segment (start 196.596 138.684) (end 196.596 137.16) (width 0.75) (layer F.Cu) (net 5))
 (segment (start 196.596 137.16) (end 202.692 131.064) (width 0.5) (layer F.Cu) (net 5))
 (segment (start 202.692 131.064) (end 202.692 108.712) (width 0.5) (layer F.Cu) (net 5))
 (segment (start 202.692 108.712) (end 200.406 106.426) (width 0.5) (layer F.Cu) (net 5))
 (segment (start 194.23 106.426) (end 191.69 108.966) (width 0.75) (layer F.Cu) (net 5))
 (segment (start 200.406 106.426) (end 194.23 106.426) (width 0.75) (layer F.Cu) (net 5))
 (segment (start 188.214 147.066) (end 196.596 138.684) (width 0.75) (layer F.Cu) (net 5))
 (segment (start 186.022 147.066) (end 188.214 147.066) (width 0.75) (layer F.Cu) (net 5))
 (segment (start 138.176 105.41) (end 142.748 109.982) (width 0.75) (layer B.Cu) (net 1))
 (segment (start 130.81 105.41) (end 138.176 105.41) (width 0.75) (layer B.Cu) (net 1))
 (segment (start 142.748 109.982) (end 142.748 103.886) (width 0.75) (layer F.Cu) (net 1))
 (segment (start 142.748 103.886) (end 139.7 100.838) (width 0.75) (layer F.Cu) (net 1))
 (segment (start 139.7 100.838) (end 139.7 98.552) (width 0.75) (layer F.Cu) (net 1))
 (segment (start 139.7 98.552) (end 141.986 96.266) (width 0.75) (layer F.Cu) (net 1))
 (segment (start 141.986 96.266) (end 183.134 96.266) (width 0.75) (layer F.Cu) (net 1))
 (segment (start 186.69 99.822) (end 186.69 108.966) (width 0.75) (layer F.Cu) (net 1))
 (segment (start 183.134 96.266) (end 186.69 99.822) (width 0.75) (layer F.Cu) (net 1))
 (segment (start 201.596 138.684) (end 201.596 133.43) (width 0.75) (layer F.Cu) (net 1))
 (segment (start 201.596 133.43) (end 203.454 131.572) (width 0.75) (layer F.Cu) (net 1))
 (segment (start 203.454 131.572) (end 203.454 107.442) (width 0.5) (layer F.Cu) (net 1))
 (segment (start 203.454 107.442) (end 201.422 105.41) (width 0.75) (layer F.Cu) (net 1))
 (segment (start 190.246 105.41) (end 186.69 108.966) (width 0.75) (layer F.Cu) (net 1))
 (segment (start 201.422 105.41) (end 190.246 105.41) (width 0.75) (layer F.Cu) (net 1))
 (via (at 142.748 109.982) (size 0.8) (drill 0.4) (layers F.Cu B.Cu) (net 1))
 (segment (start 124.238 141.5) (end 124.238 126.714) (width 0.75) (layer F.Cu) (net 1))
 (segment (start 124.238 126.714) (end 137.414 113.538) (width 0.75) (layer F.Cu) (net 1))
 (segment (start 137.414 113.538) (end 138.176 113.538) (width 0.75) (layer F.Cu) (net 1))
 (via (at 138.176 113.538) (size 0.8) (drill 0.4) (layers F.Cu B.Cu) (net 1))
 (segment (start 139.192 113.538) (end 142.748 109.982) (width 0.75) (layer B.Cu) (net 1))
 (segment (start 138.176 113.538) (end 139.192 113.538) (width 0.75) (layer B.Cu) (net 1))
 (segment (start 130.81 100.41) (end 133.938 100.41) (width 0.75) (layer F.Cu) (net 15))
 (segment (start 139.542 106.014) (end 139.542 121.69) (width 0.75) (layer F.Cu) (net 15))
 (segment (start 133.938 100.41) (end 139.542 106.014) (width 0.75) (layer F.Cu) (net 15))
 (segment (start 139.542 121.69) (end 146.328 121.69) (width 0.75) (layer B.Cu) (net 15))
 (segment (start 171.704 147.066) (end 176.022 147.066) (width 0.75) (layer B.Cu) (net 15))
 (segment (start 146.328 121.69) (end 171.704 147.066) (width 0.75) (layer B.Cu) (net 15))
 (segment (start 196.072 125.46) (end 201.168 125.46) (width 0.75) (layer F.Cu) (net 11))
 (segment (start 195.58 124.968) (end 196.072 125.46) (width 0.75) (layer F.Cu) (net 11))
 (segment (start 196.088 129.54) (end 197.358 129.54) (width 0.75) (layer F.Cu) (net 13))
 (segment (start 197.358 129.54) (end 198.12 128.778) (width 0.75) (layer F.Cu) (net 13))
 (segment (start 200.39 128.778) (end 200.914 129.302) (width 0.75) (layer F.Cu) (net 13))
 (segment (start 198.12 128.778) (end 200.39 128.778) (width 0.75) (layer F.Cu) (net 13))
 (segment (start 195.326 120.65) (end 196.596 120.65) (width 0.75) (layer F.Cu) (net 12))
 (segment (start 198.104 119.142) (end 201.422 119.142) (width 0.75) (layer F.Cu) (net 12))
 (segment (start 196.596 120.65) (end 198.104 119.142) (width 0.75) (layer F.Cu) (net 12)))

